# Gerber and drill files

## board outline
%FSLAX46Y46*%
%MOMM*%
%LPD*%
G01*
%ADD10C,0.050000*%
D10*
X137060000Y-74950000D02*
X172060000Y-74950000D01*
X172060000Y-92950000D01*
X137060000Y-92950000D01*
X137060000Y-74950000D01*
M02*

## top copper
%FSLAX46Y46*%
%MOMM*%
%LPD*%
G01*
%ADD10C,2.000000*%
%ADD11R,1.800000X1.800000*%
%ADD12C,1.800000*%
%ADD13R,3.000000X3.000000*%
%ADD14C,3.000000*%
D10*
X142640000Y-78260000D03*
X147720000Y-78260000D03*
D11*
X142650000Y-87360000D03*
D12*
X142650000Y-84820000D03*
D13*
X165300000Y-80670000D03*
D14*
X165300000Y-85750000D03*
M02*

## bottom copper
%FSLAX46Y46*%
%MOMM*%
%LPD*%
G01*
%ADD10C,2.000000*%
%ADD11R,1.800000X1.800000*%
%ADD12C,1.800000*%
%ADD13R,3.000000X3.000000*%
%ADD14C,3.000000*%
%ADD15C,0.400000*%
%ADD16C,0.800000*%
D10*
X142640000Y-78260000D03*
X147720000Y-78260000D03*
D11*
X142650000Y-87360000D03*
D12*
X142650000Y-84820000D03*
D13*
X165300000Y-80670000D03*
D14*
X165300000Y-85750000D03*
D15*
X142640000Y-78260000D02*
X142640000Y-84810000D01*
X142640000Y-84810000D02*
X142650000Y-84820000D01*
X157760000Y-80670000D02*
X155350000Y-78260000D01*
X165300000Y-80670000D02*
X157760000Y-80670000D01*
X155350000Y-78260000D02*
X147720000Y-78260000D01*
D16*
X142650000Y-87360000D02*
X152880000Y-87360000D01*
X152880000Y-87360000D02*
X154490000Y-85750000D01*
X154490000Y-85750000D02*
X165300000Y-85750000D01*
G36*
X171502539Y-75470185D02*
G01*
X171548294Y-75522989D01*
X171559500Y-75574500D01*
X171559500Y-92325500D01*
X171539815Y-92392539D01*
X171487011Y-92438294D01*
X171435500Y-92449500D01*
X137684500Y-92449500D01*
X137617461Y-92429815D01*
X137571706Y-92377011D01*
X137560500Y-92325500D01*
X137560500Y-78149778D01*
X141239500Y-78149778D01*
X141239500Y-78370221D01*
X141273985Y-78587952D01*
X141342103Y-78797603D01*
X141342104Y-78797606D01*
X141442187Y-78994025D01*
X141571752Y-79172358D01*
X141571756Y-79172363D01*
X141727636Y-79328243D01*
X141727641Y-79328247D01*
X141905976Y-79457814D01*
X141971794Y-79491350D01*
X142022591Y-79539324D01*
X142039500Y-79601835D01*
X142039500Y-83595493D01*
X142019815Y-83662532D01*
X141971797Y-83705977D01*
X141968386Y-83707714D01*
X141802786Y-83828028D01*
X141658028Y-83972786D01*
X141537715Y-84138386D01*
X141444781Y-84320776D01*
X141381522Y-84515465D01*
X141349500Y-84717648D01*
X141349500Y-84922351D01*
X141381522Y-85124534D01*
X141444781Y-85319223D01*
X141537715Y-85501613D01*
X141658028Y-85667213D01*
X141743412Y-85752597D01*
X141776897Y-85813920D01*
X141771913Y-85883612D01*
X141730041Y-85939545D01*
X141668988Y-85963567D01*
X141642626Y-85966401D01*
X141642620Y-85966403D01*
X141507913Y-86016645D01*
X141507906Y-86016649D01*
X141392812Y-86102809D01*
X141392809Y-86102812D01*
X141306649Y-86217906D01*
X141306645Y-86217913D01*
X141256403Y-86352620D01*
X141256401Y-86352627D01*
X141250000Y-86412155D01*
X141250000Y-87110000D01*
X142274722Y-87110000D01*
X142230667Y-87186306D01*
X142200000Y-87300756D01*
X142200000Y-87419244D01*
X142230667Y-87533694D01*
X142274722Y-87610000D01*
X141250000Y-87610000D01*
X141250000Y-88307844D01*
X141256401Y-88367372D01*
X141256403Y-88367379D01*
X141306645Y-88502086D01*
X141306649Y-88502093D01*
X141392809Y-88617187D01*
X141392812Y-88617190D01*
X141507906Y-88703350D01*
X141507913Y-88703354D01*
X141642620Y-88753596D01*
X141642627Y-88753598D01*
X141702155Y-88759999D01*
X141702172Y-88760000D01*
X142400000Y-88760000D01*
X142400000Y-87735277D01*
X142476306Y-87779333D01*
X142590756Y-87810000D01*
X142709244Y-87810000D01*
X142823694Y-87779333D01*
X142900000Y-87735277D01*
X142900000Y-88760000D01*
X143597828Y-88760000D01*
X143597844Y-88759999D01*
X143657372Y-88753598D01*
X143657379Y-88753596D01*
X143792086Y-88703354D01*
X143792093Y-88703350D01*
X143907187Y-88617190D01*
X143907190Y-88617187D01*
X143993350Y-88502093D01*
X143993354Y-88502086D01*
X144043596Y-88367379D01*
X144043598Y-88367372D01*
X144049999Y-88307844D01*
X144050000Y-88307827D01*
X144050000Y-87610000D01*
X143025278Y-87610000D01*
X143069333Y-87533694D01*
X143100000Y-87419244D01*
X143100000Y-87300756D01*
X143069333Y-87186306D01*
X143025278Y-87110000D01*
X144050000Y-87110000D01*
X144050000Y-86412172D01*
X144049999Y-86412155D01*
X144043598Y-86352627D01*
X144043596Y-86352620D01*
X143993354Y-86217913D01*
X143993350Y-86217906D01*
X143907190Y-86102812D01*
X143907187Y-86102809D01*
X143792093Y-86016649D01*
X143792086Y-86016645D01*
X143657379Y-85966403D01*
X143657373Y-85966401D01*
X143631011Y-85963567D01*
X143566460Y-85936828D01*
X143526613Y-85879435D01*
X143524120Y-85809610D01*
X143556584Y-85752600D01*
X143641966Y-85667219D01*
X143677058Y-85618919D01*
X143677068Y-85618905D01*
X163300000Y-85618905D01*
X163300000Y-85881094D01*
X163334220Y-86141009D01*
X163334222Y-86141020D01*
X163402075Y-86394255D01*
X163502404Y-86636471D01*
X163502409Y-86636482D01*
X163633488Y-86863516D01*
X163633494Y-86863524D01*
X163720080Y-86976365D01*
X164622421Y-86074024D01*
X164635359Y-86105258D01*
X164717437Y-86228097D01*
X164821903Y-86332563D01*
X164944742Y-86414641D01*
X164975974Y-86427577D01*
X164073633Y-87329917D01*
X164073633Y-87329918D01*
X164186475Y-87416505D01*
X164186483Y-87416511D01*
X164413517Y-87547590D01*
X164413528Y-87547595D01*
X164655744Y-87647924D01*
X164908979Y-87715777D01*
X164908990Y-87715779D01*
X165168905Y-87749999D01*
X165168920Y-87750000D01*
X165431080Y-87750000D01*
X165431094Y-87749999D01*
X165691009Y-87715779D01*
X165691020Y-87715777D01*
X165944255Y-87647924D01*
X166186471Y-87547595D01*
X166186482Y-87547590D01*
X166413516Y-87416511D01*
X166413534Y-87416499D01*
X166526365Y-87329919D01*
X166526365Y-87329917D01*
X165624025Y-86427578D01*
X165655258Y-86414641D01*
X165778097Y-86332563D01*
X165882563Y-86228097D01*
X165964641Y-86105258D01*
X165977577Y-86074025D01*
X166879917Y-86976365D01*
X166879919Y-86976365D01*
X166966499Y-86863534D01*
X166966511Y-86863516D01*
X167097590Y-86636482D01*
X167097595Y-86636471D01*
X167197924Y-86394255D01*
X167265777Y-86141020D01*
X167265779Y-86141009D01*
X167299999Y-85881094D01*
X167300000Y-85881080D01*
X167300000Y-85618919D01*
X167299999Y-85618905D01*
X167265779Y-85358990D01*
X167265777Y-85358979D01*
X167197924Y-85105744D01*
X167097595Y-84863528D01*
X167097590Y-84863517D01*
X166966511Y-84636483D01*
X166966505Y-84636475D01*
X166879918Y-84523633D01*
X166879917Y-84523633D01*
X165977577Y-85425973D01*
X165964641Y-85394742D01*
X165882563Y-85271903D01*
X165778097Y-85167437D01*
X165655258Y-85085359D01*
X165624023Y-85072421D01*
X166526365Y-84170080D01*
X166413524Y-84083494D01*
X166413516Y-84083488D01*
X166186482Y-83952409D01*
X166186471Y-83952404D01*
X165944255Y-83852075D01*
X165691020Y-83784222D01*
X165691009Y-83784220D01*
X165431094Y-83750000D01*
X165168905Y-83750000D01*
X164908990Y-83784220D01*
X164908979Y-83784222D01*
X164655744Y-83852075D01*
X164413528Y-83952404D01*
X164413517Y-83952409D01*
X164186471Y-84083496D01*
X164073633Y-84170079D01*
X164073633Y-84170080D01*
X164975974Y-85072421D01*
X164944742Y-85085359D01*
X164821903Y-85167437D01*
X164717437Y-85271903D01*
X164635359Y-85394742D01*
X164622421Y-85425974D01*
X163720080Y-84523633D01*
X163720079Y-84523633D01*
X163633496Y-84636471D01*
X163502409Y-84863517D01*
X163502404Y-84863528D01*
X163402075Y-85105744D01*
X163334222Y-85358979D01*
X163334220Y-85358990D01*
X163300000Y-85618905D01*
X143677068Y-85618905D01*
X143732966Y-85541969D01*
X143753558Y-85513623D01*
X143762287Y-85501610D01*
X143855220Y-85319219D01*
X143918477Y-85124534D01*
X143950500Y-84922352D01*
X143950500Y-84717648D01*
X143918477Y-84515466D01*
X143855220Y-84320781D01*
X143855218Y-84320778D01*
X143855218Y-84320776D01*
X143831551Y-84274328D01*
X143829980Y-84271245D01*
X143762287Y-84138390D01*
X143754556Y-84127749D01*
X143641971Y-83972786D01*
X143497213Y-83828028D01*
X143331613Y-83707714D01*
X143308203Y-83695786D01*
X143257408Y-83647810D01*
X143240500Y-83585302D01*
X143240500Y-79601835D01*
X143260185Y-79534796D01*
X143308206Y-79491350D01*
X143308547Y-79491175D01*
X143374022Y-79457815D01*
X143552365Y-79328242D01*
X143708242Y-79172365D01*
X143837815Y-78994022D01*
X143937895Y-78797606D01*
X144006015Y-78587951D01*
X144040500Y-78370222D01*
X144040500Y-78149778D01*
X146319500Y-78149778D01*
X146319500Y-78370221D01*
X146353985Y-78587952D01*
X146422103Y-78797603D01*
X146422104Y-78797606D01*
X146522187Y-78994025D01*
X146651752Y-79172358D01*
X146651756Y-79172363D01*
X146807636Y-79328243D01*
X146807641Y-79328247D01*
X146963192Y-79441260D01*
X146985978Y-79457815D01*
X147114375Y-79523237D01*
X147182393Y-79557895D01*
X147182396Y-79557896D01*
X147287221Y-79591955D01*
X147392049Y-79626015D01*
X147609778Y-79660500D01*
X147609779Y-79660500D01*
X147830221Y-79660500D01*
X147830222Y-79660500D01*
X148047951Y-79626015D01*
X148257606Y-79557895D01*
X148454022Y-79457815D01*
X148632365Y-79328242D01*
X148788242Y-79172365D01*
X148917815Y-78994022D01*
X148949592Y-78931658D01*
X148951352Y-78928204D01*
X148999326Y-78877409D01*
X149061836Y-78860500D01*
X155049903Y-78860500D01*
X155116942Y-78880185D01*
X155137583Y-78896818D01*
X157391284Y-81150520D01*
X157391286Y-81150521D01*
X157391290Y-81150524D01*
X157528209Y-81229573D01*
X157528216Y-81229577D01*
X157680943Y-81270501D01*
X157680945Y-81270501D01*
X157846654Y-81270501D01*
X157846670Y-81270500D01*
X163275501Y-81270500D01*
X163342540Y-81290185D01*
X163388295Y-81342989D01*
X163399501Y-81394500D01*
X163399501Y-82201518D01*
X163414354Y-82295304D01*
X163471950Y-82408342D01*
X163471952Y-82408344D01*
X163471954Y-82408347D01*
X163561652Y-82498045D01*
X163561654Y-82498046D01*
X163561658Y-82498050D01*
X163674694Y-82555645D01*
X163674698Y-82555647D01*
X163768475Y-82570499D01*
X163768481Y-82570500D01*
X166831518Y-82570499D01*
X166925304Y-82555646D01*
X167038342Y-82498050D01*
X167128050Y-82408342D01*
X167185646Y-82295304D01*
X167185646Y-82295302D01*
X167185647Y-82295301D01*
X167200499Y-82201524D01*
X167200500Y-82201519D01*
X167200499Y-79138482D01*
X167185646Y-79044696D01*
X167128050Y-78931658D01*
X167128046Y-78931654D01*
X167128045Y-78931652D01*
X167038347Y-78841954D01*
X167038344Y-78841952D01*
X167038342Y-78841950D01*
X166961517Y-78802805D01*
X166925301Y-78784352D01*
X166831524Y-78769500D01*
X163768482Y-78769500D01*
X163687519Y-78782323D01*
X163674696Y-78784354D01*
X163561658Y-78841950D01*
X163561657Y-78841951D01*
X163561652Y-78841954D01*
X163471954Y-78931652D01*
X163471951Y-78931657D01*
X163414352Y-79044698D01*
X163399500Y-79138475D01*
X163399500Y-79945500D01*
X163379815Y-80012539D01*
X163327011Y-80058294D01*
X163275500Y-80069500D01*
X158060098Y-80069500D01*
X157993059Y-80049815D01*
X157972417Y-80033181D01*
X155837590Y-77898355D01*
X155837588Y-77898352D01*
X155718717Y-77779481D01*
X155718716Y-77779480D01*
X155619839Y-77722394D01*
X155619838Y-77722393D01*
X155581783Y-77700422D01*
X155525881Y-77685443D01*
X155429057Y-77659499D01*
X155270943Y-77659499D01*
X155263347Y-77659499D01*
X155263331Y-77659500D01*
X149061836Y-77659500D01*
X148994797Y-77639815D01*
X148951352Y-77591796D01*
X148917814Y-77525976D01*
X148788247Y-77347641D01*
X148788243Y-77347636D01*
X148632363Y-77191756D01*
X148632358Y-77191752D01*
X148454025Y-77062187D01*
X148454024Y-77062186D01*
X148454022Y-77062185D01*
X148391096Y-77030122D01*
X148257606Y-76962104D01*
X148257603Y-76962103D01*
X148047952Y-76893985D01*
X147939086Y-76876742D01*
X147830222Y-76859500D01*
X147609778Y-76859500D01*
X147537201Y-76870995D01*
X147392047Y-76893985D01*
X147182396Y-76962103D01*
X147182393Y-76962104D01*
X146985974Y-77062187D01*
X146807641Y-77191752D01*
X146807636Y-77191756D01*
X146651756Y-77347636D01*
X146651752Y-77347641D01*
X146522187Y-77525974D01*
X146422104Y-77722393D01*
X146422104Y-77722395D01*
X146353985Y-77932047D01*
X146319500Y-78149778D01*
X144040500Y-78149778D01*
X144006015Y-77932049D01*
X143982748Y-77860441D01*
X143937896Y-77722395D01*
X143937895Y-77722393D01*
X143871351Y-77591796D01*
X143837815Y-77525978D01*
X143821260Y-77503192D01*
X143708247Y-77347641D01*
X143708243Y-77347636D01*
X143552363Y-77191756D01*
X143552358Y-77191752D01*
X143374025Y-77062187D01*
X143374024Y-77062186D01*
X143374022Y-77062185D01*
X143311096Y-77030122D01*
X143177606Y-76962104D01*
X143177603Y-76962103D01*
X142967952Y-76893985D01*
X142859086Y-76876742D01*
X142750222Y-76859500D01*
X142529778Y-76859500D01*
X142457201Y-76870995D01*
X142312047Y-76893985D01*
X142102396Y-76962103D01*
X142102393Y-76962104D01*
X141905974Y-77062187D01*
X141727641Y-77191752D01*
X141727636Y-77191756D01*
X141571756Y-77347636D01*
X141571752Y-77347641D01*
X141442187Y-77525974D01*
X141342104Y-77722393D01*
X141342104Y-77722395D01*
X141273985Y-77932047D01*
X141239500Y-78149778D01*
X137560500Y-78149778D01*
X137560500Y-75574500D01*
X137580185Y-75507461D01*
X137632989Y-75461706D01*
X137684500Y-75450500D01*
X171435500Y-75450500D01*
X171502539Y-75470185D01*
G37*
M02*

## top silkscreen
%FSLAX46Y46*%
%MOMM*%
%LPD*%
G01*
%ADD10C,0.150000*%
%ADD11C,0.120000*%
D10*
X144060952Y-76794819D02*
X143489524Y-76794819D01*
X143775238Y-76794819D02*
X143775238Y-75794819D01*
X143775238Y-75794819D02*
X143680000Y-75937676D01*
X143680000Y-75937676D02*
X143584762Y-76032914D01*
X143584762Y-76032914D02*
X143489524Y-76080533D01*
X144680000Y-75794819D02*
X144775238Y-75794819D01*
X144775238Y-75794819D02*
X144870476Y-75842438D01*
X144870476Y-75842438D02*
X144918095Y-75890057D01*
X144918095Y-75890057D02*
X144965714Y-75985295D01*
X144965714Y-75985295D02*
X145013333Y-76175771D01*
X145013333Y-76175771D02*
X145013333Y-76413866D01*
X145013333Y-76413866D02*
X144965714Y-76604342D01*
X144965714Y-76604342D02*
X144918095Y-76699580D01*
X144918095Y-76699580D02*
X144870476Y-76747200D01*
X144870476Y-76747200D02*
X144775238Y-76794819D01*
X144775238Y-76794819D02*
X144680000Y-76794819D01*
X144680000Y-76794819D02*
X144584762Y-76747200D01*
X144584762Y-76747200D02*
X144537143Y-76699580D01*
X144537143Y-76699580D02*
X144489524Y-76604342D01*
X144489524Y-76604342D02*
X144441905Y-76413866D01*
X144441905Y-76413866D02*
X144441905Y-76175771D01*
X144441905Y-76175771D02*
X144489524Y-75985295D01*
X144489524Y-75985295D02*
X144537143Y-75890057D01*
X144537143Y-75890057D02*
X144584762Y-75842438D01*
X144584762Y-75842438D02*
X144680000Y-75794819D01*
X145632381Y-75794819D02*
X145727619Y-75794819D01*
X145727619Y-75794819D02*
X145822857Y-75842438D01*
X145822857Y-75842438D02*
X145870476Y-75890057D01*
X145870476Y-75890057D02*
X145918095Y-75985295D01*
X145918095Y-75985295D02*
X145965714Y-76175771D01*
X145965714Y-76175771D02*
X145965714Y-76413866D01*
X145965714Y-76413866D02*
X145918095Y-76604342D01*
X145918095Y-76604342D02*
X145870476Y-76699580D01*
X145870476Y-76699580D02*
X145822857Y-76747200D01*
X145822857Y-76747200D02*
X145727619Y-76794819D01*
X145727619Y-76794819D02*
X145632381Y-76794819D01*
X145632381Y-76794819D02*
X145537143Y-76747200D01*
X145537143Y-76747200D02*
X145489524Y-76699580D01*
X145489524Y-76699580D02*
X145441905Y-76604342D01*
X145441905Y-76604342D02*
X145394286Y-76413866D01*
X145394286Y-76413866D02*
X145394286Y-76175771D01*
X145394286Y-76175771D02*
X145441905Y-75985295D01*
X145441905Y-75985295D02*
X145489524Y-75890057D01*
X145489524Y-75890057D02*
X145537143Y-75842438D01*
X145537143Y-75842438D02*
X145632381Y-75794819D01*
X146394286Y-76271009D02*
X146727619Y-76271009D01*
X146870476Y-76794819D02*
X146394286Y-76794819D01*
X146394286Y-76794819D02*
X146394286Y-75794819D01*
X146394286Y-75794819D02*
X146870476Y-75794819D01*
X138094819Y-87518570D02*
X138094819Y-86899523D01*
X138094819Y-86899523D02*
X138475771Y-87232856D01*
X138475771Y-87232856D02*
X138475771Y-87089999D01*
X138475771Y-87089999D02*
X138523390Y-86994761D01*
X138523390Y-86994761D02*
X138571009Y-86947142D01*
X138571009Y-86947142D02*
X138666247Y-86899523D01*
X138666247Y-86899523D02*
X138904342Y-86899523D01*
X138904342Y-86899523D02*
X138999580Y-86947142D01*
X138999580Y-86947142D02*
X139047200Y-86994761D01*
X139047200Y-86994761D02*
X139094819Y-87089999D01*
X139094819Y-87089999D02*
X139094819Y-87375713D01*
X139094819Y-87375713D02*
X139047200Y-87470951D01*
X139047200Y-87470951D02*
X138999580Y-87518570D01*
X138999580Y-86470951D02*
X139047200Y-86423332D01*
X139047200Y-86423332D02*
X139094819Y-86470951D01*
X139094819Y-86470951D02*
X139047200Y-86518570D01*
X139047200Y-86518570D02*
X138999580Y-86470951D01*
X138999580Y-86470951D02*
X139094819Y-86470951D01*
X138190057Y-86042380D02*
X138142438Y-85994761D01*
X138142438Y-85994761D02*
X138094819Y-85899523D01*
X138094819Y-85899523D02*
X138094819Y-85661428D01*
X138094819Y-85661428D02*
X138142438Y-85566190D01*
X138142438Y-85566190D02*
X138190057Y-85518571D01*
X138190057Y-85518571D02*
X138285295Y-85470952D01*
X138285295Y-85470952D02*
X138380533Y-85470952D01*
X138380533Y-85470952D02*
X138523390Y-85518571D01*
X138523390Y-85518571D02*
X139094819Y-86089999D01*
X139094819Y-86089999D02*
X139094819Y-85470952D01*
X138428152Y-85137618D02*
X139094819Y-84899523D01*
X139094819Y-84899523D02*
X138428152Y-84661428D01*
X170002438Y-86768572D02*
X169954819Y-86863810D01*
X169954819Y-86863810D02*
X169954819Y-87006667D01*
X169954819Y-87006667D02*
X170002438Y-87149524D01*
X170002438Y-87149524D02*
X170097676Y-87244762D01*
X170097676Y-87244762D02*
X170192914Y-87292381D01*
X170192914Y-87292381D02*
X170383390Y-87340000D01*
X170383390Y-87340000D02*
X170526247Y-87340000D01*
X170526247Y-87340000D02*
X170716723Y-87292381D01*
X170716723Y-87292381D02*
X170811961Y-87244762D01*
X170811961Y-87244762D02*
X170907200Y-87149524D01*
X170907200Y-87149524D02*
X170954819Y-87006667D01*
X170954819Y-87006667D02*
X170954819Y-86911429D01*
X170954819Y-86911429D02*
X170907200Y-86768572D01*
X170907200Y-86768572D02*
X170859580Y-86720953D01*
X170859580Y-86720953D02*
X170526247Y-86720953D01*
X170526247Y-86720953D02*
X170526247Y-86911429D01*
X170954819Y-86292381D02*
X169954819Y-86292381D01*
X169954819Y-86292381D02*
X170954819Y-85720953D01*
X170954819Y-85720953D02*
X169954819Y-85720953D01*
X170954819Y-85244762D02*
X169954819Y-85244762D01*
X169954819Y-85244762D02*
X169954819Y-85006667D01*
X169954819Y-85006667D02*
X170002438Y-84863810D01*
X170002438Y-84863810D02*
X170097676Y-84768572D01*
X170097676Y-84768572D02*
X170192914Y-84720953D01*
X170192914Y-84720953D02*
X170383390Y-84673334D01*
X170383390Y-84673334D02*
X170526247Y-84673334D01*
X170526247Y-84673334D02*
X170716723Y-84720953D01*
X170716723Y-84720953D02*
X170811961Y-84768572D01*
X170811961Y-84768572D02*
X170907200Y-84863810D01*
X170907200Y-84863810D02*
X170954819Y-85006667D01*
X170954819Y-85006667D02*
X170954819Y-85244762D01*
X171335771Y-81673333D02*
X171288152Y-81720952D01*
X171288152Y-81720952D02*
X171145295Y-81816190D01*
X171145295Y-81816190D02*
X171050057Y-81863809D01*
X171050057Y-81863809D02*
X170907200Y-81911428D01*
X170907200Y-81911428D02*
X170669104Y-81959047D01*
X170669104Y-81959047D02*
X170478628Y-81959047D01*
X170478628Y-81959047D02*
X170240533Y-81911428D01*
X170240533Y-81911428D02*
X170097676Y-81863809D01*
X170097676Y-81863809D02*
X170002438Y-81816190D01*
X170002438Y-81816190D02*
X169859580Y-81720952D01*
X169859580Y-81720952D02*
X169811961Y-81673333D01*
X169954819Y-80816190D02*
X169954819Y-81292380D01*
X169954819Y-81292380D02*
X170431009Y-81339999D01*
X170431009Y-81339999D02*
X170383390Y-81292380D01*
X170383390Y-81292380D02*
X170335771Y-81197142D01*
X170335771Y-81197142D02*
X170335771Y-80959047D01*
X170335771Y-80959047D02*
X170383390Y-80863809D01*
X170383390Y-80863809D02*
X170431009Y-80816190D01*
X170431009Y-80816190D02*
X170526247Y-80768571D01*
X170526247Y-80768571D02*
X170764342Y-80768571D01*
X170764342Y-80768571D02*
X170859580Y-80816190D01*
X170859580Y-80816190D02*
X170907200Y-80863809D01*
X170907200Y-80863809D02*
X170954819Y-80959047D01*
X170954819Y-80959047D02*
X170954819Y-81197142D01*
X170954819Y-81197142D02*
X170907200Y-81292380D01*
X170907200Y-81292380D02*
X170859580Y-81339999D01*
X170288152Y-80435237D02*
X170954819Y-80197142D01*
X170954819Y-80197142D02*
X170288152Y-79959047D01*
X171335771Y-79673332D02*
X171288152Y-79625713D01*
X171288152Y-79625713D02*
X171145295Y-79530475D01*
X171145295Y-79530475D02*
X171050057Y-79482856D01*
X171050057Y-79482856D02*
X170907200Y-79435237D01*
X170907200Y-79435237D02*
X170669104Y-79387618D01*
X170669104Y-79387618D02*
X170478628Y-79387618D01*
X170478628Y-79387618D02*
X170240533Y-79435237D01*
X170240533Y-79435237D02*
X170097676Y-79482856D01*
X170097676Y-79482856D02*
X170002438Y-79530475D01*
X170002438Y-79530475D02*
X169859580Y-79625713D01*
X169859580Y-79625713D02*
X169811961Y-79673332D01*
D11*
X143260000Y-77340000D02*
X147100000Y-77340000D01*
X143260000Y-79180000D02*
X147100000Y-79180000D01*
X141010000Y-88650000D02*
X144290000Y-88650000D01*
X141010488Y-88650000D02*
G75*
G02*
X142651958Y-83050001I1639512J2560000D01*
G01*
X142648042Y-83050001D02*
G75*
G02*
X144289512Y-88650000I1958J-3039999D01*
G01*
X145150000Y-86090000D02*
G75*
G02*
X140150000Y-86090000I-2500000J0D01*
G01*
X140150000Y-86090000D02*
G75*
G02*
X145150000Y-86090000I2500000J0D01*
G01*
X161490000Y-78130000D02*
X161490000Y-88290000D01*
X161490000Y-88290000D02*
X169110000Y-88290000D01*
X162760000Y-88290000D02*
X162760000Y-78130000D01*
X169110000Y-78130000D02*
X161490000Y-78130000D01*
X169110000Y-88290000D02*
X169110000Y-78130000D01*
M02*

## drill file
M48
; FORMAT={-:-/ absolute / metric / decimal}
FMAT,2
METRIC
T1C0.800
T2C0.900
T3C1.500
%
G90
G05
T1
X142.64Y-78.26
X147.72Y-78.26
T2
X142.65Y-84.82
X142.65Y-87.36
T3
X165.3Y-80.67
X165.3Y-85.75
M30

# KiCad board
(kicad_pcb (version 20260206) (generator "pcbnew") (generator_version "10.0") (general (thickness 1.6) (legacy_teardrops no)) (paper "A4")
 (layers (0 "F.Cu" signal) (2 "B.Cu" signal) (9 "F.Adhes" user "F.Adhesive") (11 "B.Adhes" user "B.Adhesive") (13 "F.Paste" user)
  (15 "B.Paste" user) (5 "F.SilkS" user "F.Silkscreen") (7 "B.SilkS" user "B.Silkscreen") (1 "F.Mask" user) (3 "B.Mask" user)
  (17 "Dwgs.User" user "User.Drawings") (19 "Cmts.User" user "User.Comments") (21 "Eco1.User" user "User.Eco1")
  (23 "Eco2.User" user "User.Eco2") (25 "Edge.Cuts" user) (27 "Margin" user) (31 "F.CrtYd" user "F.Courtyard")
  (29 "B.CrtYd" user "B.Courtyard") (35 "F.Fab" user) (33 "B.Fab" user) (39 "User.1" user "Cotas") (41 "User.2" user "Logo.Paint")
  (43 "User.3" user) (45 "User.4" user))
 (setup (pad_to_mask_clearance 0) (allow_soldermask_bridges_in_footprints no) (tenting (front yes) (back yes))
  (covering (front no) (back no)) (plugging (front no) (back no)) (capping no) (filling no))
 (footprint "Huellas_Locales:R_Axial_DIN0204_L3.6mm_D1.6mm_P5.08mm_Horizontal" (layer "F.Cu") (at 142.64 78.26)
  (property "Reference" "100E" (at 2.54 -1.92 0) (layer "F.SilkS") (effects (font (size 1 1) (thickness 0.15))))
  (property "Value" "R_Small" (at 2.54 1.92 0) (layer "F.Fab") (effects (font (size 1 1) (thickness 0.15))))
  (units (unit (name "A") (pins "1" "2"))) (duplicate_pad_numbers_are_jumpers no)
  (fp_line (start 0.62 -0.92) (end 4.46 -0.92) (stroke (width 0.12) (type solid)) (layer "F.SilkS"))
  (fp_line (start 0.62 0.92) (end 4.46 0.92) (stroke (width 0.12) (type solid)) (layer "F.SilkS"))
  (pad "1" thru_hole circle (at 0 0) (size 2 2) (drill 0.8) (layers "*.Cu" "*.Mask") (remove_unused_layers no) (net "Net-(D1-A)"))
  (pad "2" thru_hole circle (at 5.08 0) (size 2 2) (drill 0.8) (layers "*.Cu" "*.Mask") (remove_unused_layers no) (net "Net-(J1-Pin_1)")))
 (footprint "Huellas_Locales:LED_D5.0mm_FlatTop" (layer "F.Cu") (at 142.65 87.36 90)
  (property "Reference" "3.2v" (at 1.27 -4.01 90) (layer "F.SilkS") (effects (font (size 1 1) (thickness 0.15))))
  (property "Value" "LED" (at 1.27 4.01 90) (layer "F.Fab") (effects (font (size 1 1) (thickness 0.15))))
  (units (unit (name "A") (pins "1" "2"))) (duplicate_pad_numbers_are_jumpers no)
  (fp_line (start -1.29 -1.64) (end -1.29 1.64) (stroke (width 0.12) (type solid)) (layer "F.SilkS"))
  (fp_arc (start -1.29 -1.639512) (mid 2.125106 -2.917258) (end 4.309999 0.001958) (stroke (width 0.12) (type solid)) (layer "F.SilkS"))
  (fp_arc (start 4.309999 -0.001958) (mid 2.125106 2.917258) (end -1.29 1.639512) (stroke (width 0.12) (type solid)) (layer "F.SilkS"))
  (fp_circle (center 1.27 0) (end 3.77 0) (stroke (width 0.12) (type solid)) (fill no) (layer "F.SilkS"))
  (pad "1" thru_hole rect (at 0 0 90) (size 1.8 1.8) (drill 0.9) (layers "*.Cu" "*.Mask") (remove_unused_layers no) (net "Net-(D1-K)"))
  (pad "2" thru_hole circle (at 2.54 0 90) (size 1.8 1.8) (drill 0.9) (layers "*.Cu" "*.Mask") (remove_unused_layers no) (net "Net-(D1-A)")))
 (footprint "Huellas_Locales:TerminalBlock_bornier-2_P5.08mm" (layer "F.Cu") (at 165.3 80.67 -90)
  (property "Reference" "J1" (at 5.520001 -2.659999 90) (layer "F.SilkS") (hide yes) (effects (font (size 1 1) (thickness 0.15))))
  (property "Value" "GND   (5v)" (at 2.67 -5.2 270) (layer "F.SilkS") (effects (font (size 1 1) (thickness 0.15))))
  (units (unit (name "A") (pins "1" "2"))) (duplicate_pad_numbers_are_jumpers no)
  (fp_line (start -2.54 3.81) (end 7.62 3.81) (stroke (width 0.12) (type solid)) (layer "F.SilkS"))
  (fp_line (start 7.62 3.81) (end 7.62 -3.81) (stroke (width 0.12) (type solid)) (layer "F.SilkS"))
  (fp_line (start 7.62 2.54) (end -2.54 2.54) (stroke (width 0.12) (type solid)) (layer "F.SilkS"))
  (fp_line (start -2.54 -3.81) (end -2.54 3.81) (stroke (width 0.12) (type solid)) (layer "F.SilkS"))
  (fp_line (start 7.62 -3.81) (end -2.54 -3.81) (stroke (width 0.12) (type solid)) (layer "F.SilkS"))
  (pad "1" thru_hole rect (at 0 0 270) (size 3 3) (drill 1.5) (layers "*.Cu" "*.Mask") (remove_unused_layers no) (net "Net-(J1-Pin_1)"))
  (pad "2" thru_hole circle (at 5.08 0 270) (size 3 3) (drill 1.5) (layers "*.Cu" "*.Mask") (remove_unused_layers no) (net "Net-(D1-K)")))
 (gr_rect (start 137.06 74.95) (end 172.06 92.95) (stroke (width 0.05) (type default)) (fill no) (layer "Edge.Cuts"))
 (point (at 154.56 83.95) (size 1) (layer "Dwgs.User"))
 (segment (start 142.64 78.26) (end 142.64 84.81) (width 0.4) (layer "B.Cu") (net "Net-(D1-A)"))
 (segment (start 142.64 84.81) (end 142.65 84.82) (width 0.4) (layer "B.Cu") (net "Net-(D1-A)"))
 (segment (start 157.76 80.67) (end 155.35 78.26) (width 0.4) (layer "B.Cu") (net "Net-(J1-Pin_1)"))
 (segment (start 165.3 80.67) (end 157.76 80.67) (width 0.4) (layer "B.Cu") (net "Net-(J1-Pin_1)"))
 (segment (start 155.35 78.26) (end 147.72 78.26) (width 0.4) (layer "B.Cu") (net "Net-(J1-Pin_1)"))
 (segment (start 142.65 87.36) (end 152.88 87.36) (width 0.8) (layer "B.Cu") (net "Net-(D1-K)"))
 (segment (start 152.88 87.36) (end 154.49 85.75) (width 0.8) (layer "B.Cu") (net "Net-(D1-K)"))
 (segment (start 154.49 85.75) (end 165.3 85.75) (width 0.8) (layer "B.Cu") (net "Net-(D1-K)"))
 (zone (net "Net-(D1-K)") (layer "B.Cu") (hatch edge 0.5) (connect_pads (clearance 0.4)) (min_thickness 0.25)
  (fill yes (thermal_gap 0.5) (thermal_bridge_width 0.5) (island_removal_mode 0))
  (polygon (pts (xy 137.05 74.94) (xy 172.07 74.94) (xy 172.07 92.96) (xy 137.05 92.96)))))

